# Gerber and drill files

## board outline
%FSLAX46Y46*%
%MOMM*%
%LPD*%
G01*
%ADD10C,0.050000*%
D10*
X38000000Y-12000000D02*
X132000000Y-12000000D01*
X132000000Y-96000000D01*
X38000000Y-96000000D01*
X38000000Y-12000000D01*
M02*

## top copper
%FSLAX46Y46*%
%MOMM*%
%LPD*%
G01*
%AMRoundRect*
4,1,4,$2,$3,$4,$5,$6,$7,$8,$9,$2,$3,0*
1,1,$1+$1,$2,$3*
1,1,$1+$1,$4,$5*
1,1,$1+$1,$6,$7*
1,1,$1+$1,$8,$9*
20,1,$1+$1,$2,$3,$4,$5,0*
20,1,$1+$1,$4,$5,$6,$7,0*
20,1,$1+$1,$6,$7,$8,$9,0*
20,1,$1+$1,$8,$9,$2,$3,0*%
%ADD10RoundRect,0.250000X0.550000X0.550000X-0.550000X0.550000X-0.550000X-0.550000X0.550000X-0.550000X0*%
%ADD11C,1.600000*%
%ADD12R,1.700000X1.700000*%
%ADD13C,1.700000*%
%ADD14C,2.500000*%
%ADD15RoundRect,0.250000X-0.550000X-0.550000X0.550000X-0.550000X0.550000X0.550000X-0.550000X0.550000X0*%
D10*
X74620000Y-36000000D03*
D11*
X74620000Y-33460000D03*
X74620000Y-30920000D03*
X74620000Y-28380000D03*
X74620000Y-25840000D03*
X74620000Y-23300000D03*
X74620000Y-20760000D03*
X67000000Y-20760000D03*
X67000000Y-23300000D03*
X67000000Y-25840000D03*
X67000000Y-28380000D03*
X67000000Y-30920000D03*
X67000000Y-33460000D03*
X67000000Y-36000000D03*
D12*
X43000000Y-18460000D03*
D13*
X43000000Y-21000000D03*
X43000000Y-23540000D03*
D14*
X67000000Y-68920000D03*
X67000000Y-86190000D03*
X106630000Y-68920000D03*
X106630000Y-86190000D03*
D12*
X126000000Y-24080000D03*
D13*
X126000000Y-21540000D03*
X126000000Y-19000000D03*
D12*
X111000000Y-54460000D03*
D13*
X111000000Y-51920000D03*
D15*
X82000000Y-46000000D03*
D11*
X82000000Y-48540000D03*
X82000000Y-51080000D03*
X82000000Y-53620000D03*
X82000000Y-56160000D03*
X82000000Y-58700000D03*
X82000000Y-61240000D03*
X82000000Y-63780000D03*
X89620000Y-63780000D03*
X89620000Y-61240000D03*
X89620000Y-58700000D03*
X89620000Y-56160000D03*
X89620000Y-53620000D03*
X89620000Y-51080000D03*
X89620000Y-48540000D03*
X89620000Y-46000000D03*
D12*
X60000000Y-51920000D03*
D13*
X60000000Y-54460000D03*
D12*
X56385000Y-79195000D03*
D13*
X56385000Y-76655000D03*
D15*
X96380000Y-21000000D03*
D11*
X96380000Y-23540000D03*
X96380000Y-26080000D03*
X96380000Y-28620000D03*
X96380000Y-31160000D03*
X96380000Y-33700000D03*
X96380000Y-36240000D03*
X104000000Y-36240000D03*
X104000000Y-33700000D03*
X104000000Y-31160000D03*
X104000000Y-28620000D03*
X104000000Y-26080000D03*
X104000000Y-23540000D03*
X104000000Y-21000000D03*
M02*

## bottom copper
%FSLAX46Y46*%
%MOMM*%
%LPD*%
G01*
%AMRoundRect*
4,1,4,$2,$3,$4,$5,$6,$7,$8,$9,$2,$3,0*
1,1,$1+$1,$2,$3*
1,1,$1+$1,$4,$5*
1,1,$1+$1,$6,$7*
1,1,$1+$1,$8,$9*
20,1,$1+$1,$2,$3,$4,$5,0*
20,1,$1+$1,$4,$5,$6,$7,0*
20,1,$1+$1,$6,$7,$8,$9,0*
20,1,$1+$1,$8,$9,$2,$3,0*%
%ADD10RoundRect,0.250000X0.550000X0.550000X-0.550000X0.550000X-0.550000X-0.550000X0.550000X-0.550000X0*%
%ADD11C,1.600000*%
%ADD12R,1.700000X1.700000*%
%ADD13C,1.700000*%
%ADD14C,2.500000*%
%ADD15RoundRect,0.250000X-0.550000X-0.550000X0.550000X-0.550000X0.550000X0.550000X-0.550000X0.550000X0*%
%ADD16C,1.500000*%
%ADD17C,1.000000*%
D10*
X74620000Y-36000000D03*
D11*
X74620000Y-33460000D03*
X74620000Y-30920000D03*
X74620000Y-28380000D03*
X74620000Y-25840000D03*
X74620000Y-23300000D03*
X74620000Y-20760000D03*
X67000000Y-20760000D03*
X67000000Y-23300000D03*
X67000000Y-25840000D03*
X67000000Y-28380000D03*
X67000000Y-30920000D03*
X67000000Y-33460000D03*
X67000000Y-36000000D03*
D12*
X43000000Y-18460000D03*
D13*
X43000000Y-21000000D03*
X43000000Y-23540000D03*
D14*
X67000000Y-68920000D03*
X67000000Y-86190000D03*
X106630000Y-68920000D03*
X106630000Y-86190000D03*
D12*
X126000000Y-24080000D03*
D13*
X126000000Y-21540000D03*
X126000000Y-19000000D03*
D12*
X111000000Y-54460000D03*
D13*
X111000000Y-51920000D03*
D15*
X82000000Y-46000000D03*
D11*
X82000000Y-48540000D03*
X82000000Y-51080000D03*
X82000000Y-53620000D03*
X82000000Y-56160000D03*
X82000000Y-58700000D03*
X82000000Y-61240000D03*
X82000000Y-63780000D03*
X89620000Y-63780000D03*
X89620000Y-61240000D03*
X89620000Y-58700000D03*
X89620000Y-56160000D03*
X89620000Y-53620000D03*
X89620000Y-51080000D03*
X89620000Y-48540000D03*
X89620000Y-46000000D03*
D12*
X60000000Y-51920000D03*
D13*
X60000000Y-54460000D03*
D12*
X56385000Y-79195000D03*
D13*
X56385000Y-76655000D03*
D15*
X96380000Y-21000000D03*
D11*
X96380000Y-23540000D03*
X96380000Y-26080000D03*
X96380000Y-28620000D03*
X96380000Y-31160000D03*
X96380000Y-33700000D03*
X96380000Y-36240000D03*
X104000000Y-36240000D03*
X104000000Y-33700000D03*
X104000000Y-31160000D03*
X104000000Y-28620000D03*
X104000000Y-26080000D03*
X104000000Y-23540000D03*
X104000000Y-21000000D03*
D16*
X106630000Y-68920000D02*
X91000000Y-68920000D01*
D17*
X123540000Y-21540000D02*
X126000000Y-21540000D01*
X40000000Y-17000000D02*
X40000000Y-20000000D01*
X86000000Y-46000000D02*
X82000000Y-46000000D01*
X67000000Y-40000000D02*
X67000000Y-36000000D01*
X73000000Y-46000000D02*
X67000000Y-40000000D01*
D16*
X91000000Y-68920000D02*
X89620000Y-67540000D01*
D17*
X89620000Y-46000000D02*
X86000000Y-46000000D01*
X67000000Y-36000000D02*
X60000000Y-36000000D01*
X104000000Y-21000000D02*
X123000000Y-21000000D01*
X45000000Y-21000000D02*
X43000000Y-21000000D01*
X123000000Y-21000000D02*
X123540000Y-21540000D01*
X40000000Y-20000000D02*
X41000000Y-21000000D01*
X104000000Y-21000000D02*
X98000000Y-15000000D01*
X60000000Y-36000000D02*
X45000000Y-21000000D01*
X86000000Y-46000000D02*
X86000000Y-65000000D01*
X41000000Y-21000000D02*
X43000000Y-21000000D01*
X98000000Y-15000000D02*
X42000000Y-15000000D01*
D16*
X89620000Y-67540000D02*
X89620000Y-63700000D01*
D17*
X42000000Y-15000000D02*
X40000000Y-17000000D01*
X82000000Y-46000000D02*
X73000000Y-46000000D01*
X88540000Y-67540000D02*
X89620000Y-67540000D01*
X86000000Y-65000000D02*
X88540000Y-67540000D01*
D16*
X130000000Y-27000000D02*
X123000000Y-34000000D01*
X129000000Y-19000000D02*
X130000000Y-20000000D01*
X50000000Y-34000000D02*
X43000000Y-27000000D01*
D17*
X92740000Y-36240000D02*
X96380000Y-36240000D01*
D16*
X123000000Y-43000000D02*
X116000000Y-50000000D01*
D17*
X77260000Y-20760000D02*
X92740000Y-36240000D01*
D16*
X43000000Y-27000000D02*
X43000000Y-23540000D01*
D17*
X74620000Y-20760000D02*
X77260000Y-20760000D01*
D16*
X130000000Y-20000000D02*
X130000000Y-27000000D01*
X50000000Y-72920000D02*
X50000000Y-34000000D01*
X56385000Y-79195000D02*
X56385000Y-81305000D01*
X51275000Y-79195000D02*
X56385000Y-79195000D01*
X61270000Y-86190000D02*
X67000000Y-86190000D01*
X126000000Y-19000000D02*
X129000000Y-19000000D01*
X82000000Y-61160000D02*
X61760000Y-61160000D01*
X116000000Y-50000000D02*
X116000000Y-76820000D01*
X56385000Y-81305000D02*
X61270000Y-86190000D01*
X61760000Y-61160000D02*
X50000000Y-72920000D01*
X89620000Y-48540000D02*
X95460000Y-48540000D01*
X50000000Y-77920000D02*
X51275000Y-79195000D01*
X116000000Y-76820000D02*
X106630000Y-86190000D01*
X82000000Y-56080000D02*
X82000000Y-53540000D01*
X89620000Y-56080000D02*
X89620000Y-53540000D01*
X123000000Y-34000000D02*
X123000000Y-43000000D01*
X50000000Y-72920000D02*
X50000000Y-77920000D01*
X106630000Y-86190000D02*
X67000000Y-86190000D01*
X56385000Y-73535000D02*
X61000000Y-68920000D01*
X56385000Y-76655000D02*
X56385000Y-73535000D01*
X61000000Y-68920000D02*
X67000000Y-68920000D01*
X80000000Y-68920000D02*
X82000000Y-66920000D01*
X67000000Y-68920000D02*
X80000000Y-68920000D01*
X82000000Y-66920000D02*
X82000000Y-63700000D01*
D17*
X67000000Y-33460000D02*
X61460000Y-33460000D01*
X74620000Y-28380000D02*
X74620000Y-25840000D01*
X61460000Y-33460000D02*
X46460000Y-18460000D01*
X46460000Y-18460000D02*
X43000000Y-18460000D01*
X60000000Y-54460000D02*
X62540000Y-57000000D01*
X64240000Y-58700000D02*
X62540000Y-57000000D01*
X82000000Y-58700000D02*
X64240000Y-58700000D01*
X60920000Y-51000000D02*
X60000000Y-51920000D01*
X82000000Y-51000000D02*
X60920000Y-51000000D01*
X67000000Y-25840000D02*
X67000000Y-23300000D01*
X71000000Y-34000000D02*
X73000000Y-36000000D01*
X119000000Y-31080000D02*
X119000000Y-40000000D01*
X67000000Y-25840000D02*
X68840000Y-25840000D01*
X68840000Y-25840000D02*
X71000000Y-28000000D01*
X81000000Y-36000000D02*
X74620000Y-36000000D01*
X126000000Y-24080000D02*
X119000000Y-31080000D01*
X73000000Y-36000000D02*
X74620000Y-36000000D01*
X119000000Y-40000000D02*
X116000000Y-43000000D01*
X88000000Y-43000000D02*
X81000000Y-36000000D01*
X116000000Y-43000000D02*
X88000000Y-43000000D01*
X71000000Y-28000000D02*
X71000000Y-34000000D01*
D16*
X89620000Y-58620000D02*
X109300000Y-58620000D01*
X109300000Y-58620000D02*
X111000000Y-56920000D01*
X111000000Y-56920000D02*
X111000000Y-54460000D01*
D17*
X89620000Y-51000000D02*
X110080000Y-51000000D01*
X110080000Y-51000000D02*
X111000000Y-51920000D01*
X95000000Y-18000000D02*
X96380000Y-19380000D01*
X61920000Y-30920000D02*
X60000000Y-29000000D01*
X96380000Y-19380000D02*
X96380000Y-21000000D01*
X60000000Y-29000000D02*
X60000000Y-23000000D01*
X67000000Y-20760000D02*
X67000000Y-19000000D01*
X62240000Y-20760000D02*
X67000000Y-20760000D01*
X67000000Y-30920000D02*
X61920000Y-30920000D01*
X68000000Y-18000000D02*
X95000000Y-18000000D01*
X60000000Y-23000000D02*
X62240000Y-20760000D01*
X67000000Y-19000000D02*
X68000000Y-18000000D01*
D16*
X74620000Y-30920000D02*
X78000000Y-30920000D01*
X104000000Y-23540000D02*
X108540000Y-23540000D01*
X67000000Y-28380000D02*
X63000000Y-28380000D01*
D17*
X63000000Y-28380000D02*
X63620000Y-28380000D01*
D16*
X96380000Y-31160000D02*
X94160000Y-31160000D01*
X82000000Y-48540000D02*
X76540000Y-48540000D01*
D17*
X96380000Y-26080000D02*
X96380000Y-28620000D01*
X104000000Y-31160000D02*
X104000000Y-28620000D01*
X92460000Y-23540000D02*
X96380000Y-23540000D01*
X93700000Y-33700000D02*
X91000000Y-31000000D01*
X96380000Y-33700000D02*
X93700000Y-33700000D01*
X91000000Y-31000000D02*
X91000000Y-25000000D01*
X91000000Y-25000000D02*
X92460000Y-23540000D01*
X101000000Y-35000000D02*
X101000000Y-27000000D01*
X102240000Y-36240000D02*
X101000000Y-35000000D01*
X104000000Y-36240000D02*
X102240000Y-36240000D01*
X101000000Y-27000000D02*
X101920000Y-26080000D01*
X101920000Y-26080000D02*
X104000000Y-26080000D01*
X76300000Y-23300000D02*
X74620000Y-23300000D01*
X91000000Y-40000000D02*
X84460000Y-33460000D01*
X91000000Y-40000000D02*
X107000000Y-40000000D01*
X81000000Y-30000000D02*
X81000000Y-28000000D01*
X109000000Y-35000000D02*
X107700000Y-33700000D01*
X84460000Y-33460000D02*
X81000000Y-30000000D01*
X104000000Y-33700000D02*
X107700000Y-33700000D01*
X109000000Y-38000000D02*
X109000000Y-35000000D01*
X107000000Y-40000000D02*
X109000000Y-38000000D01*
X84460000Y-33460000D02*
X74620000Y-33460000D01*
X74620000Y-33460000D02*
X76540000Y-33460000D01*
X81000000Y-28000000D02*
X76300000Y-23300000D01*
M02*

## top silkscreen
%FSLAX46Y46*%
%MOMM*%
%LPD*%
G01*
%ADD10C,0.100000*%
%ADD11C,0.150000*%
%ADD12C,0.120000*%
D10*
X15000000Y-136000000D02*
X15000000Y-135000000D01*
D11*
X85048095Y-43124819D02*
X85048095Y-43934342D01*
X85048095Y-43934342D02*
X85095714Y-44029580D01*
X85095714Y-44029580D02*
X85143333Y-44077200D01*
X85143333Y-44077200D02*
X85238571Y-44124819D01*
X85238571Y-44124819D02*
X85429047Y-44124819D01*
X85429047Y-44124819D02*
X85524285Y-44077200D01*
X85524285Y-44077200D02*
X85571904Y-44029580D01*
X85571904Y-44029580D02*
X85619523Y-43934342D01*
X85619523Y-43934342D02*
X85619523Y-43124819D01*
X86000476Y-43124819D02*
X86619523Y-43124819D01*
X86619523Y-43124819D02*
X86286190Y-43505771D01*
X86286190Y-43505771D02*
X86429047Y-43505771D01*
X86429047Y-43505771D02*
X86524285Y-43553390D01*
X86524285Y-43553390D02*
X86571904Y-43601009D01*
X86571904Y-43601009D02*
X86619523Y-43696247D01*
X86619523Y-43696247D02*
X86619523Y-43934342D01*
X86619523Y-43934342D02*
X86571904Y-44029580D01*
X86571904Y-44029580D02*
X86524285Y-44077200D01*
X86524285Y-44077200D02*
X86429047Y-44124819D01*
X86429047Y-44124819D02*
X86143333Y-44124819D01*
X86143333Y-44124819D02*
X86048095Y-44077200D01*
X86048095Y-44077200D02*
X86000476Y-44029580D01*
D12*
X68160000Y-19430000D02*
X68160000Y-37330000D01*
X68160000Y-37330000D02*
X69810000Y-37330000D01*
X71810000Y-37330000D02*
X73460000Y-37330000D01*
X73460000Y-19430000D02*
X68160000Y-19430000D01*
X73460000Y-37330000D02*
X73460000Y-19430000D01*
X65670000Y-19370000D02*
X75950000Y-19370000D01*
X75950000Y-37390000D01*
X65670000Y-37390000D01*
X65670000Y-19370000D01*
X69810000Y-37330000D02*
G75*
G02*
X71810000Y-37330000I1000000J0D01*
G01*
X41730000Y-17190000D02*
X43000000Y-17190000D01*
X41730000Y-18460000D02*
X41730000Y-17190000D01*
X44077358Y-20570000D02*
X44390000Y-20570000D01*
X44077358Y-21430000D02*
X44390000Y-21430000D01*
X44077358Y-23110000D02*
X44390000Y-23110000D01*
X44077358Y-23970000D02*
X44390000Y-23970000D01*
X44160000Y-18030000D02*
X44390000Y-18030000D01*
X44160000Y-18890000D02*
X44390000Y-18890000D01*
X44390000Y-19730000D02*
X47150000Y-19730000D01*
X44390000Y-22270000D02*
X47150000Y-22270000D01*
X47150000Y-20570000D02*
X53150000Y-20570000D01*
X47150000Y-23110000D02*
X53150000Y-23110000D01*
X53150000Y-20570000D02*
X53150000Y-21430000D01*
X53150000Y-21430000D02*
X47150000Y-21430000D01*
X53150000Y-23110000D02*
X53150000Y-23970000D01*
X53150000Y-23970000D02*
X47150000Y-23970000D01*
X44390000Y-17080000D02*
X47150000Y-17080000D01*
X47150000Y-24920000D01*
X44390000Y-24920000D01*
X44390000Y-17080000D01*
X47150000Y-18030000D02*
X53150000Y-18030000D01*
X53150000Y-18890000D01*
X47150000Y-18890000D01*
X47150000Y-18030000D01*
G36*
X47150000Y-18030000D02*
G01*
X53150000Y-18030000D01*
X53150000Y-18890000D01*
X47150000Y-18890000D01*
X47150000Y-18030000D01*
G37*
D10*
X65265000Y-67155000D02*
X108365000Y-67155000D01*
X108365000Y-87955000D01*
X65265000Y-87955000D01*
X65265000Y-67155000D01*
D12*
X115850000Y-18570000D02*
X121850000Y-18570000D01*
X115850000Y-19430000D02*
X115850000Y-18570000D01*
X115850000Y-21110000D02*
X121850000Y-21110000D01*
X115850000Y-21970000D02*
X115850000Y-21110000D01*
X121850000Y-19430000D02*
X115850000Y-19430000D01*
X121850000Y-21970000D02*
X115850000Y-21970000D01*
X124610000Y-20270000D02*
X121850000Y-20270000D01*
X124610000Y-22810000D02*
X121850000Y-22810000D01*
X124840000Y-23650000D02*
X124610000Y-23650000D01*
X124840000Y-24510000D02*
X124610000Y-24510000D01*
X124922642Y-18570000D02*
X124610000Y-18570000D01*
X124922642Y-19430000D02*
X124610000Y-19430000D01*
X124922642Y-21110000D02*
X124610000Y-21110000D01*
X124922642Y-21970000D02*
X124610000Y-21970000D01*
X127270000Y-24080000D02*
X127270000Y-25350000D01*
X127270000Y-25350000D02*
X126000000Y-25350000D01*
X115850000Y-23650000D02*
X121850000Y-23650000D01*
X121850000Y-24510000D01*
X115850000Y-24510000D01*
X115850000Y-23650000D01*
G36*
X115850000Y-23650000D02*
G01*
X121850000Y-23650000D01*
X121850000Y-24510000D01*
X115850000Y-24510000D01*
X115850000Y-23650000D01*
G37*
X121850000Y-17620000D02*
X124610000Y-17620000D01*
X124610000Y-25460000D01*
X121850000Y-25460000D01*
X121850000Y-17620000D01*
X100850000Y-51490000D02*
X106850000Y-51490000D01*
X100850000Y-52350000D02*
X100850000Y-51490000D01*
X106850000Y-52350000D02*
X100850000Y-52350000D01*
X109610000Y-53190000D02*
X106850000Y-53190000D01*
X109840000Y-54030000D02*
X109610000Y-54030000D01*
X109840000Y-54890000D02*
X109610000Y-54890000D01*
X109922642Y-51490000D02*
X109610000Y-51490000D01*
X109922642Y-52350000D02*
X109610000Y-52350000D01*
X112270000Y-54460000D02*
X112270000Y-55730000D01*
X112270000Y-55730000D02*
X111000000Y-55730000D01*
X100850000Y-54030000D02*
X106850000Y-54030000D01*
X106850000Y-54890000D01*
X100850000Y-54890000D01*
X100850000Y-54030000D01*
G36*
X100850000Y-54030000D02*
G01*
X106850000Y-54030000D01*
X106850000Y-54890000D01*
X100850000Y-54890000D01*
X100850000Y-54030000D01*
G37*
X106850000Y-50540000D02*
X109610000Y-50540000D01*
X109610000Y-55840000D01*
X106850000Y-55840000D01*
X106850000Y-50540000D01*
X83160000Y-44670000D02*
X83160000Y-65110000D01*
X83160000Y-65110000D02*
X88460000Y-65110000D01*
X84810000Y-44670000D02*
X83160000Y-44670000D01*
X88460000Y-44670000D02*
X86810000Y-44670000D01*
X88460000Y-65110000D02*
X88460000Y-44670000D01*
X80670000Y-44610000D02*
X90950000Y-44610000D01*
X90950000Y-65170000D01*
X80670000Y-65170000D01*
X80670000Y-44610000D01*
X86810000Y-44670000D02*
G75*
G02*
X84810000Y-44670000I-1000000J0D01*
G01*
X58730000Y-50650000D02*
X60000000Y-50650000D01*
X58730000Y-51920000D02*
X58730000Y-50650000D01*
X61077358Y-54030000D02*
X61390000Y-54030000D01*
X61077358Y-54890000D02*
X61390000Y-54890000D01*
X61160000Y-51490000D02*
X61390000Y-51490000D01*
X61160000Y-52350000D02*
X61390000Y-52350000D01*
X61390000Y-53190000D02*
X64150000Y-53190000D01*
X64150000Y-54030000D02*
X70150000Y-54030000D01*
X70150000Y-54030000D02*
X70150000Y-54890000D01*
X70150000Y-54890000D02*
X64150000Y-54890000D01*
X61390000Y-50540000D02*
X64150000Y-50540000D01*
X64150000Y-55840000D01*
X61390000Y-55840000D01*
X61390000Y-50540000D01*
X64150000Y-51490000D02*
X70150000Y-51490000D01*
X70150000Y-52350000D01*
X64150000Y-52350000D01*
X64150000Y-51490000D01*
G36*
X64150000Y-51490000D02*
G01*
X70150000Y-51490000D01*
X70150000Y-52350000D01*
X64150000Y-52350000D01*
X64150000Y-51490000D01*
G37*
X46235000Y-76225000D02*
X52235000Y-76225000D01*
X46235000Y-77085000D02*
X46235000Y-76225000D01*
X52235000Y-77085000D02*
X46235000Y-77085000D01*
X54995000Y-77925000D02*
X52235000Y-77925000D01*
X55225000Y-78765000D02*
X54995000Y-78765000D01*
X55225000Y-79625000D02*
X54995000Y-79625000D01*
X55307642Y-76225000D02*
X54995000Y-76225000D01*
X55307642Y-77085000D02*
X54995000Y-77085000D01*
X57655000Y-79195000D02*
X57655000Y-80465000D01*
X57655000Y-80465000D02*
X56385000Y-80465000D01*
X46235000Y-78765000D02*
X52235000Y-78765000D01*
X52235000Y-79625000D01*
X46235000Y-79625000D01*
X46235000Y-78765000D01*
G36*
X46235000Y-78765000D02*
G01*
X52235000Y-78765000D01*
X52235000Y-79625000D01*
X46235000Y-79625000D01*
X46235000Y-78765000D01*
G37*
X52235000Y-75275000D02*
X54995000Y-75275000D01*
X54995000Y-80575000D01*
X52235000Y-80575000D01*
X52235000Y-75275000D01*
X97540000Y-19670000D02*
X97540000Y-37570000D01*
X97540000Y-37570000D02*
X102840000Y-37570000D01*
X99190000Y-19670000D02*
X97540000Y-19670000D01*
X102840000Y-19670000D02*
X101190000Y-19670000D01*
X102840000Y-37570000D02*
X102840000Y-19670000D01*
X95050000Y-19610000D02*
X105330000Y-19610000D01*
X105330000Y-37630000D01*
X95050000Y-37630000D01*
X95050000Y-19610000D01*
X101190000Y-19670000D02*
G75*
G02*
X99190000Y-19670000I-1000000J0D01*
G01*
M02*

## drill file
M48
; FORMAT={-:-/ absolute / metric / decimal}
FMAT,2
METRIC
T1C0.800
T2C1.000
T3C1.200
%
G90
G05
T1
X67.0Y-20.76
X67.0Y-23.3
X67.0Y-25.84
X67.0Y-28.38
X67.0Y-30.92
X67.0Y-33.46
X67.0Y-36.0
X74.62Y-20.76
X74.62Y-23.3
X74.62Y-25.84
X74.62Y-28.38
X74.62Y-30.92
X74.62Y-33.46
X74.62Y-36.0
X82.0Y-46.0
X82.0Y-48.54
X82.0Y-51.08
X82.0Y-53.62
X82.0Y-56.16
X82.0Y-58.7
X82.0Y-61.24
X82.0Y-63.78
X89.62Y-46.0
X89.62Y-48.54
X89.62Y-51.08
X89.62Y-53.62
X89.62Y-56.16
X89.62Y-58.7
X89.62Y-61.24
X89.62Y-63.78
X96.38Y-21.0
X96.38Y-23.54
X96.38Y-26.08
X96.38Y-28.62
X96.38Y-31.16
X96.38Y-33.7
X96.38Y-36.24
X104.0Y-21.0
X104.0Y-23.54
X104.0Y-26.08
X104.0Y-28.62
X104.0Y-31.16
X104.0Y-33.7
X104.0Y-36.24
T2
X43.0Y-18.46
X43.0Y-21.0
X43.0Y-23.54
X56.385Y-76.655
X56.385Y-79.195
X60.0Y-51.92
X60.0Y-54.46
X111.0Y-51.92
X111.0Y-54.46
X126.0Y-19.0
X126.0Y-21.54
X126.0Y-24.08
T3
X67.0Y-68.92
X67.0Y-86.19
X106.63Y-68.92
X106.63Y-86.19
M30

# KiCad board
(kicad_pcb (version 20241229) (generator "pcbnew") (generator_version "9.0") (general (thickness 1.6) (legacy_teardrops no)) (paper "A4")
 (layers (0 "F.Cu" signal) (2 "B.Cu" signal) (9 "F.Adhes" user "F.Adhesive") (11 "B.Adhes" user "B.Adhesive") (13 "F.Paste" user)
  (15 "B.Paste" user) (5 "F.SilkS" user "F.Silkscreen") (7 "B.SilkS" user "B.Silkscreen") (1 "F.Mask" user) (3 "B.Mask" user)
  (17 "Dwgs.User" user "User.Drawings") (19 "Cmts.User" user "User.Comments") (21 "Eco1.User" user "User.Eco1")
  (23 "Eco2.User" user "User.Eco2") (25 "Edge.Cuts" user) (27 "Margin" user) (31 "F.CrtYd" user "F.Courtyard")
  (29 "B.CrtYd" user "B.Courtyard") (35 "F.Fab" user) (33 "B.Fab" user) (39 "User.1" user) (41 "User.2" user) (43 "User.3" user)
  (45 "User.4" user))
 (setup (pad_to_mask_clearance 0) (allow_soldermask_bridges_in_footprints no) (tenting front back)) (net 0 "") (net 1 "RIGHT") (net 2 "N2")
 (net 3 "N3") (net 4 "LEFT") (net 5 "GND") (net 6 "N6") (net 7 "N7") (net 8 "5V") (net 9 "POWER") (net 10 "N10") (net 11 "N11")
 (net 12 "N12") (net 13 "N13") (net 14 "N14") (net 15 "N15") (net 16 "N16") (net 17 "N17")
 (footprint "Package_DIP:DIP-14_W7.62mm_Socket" (layer "F.Cu") (at 74.62 36 180)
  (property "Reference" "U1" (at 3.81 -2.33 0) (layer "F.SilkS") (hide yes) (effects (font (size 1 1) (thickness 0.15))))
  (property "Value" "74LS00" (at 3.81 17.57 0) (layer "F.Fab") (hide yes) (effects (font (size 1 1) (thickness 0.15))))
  (fp_line (start 6.46 16.57) (end 6.46 -1.33) (stroke (width 0.12) (type solid)) (layer "F.SilkS"))
  (fp_line (start 6.46 -1.33) (end 4.81 -1.33) (stroke (width 0.12) (type solid)) (layer "F.SilkS"))
  (fp_line (start 2.81 -1.33) (end 1.16 -1.33) (stroke (width 0.12) (type solid)) (layer "F.SilkS"))
  (fp_line (start 1.16 16.57) (end 6.46 16.57) (stroke (width 0.12) (type solid)) (layer "F.SilkS"))
  (fp_line (start 1.16 -1.33) (end 1.16 16.57) (stroke (width 0.12) (type solid)) (layer "F.SilkS"))
  (fp_rect (start -1.33 -1.39) (end 8.95 16.63) (stroke (width 0.12) (type solid)) (fill no) (layer "F.SilkS"))
  (fp_arc (start 4.81 -1.33) (mid 3.81 -0.33) (end 2.81 -1.33) (stroke (width 0.12) (type solid)) (layer "F.SilkS"))
  (pad "1" thru_hole roundrect (at 0 0 180) (size 1.6 1.6) (drill 0.8) (layers "*.Cu" "*.Mask") (remove_unused_layers no)
   (roundrect_rratio 0.15625) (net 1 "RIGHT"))
  (pad "2" thru_hole circle (at 0 2.54 180) (size 1.6 1.6) (drill 0.8) (layers "*.Cu" "*.Mask") (remove_unused_layers no) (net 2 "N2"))
  (pad "3" thru_hole circle (at 0 5.08 180) (size 1.6 1.6) (drill 0.8) (layers "*.Cu" "*.Mask") (remove_unused_layers no) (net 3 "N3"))
  (pad "4" thru_hole circle (at 0 7.62 180) (size 1.6 1.6) (drill 0.8) (layers "*.Cu" "*.Mask") (remove_unused_layers no) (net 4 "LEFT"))
  (pad "5" thru_hole circle (at 0 10.16 180) (size 1.6 1.6) (drill 0.8) (layers "*.Cu" "*.Mask") (remove_unused_layers no) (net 4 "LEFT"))
  (pad "6" thru_hole circle (at 0 12.7 180) (size 1.6 1.6) (drill 0.8) (layers "*.Cu" "*.Mask") (remove_unused_layers no) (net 2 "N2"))
  (pad "7" thru_hole circle (at 0 15.24 180) (size 1.6 1.6) (drill 0.8) (layers "*.Cu" "*.Mask") (remove_unused_layers no) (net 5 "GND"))
  (pad "8" thru_hole circle (at 7.62 15.24 180) (size 1.6 1.6) (drill 0.8) (layers "*.Cu" "*.Mask") (remove_unused_layers no) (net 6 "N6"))
  (pad "9" thru_hole circle (at 7.62 12.7 180) (size 1.6 1.6) (drill 0.8) (layers "*.Cu" "*.Mask") (remove_unused_layers no) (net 1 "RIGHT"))
  (pad "10" thru_hole circle (at 7.62 10.16 180) (size 1.6 1.6) (drill 0.8) (layers "*.Cu" "*.Mask") (remove_unused_layers no)
   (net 1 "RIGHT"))
  (pad "11" thru_hole circle (at 7.62 7.62 180) (size 1.6 1.6) (drill 0.8) (layers "*.Cu" "*.Mask") (remove_unused_layers no) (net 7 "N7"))
  (pad "12" thru_hole circle (at 7.62 5.08 180) (size 1.6 1.6) (drill 0.8) (layers "*.Cu" "*.Mask") (remove_unused_layers no) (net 6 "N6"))
  (pad "13" thru_hole circle (at 7.62 2.54 180) (size 1.6 1.6) (drill 0.8) (layers "*.Cu" "*.Mask") (remove_unused_layers no) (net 4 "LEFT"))
  (pad "14" thru_hole circle (at 7.62 0 180) (size 1.6 1.6) (drill 0.8) (layers "*.Cu" "*.Mask") (remove_unused_layers no) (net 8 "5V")))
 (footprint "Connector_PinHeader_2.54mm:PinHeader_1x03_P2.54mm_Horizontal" (layer "F.Cu") (at 43 18.46)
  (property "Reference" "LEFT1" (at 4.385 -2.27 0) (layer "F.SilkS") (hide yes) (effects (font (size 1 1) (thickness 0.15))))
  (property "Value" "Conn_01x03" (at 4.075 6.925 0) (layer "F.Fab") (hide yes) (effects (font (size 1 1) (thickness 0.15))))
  (fp_line (start -1.27 -1.27) (end 0 -1.27) (stroke (width 0.12) (type solid)) (layer "F.SilkS"))
  (fp_line (start -1.27 0) (end -1.27 -1.27) (stroke (width 0.12) (type solid)) (layer "F.SilkS"))
  (fp_line (start 1.077358 2.11) (end 1.39 2.11) (stroke (width 0.12) (type solid)) (layer "F.SilkS"))
  (fp_line (start 1.077358 2.97) (end 1.39 2.97) (stroke (width 0.12) (type solid)) (layer "F.SilkS"))
  (fp_line (start 1.077358 4.65) (end 1.39 4.65) (stroke (width 0.12) (type solid)) (layer "F.SilkS"))
  (fp_line (start 1.077358 5.51) (end 1.39 5.51) (stroke (width 0.12) (type solid)) (layer "F.SilkS"))
  (fp_line (start 1.16 -0.43) (end 1.39 -0.43) (stroke (width 0.12) (type solid)) (layer "F.SilkS"))
  (fp_line (start 1.16 0.43) (end 1.39 0.43) (stroke (width 0.12) (type solid)) (layer "F.SilkS"))
  (fp_line (start 1.39 1.27) (end 4.15 1.27) (stroke (width 0.12) (type solid)) (layer "F.SilkS"))
  (fp_line (start 1.39 3.81) (end 4.15 3.81) (stroke (width 0.12) (type solid)) (layer "F.SilkS"))
  (fp_line (start 4.15 2.11) (end 10.15 2.11) (stroke (width 0.12) (type solid)) (layer "F.SilkS"))
  (fp_line (start 4.15 4.65) (end 10.15 4.65) (stroke (width 0.12) (type solid)) (layer "F.SilkS"))
  (fp_line (start 10.15 2.11) (end 10.15 2.97) (stroke (width 0.12) (type solid)) (layer "F.SilkS"))
  (fp_line (start 10.15 2.97) (end 4.15 2.97) (stroke (width 0.12) (type solid)) (layer "F.SilkS"))
  (fp_line (start 10.15 4.65) (end 10.15 5.51) (stroke (width 0.12) (type solid)) (layer "F.SilkS"))
  (fp_line (start 10.15 5.51) (end 4.15 5.51) (stroke (width 0.12) (type solid)) (layer "F.SilkS"))
  (fp_rect (start 1.39 -1.38) (end 4.15 6.46) (stroke (width 0.12) (type solid)) (fill no) (layer "F.SilkS"))
  (fp_rect (start 4.15 -0.43) (end 10.15 0.43) (stroke (width 0.12) (type solid)) (fill yes) (layer "F.SilkS"))
  (pad "1" thru_hole rect (at 0 0) (size 1.7 1.7) (drill 1) (layers "*.Cu" "*.Mask") (remove_unused_layers no) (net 4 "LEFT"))
  (pad "2" thru_hole circle (at 0 2.54) (size 1.7 1.7) (drill 1) (layers "*.Cu" "*.Mask") (remove_unused_layers no) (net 8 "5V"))
  (pad "3" thru_hole circle (at 0 5.08) (size 1.7 1.7) (drill 1) (layers "*.Cu" "*.Mask") (remove_unused_layers no) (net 5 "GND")))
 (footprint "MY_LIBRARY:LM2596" (layer "F.Cu") (at 67 86.19)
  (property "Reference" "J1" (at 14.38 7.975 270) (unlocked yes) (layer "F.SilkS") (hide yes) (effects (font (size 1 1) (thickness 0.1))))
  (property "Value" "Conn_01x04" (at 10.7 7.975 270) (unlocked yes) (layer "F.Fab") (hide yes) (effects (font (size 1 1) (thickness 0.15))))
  (fp_rect (start -1.735 1.765) (end 41.365 -19.035) (stroke (width 0.1) (type solid)) (fill no) (layer "F.SilkS"))
  (pad "IN+" thru_hole circle (at 0 -17.27) (size 2.5 2.5) (drill 1.2) (layers "*.Cu" "*.Mask") (remove_unused_layers no) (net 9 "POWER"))
  (pad "IN-" thru_hole circle (at 0 0) (size 2.5 2.5) (drill 1.2) (layers "*.Cu" "*.Mask") (remove_unused_layers no) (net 5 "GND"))
  (pad "OUT+" thru_hole circle (at 39.63 -17.27) (size 2.5 2.5) (drill 1.2) (layers "*.Cu" "*.Mask") (remove_unused_layers no) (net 8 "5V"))
  (pad "OUT-" thru_hole circle (at 39.63 0) (size 2.5 2.5) (drill 1.2) (layers "*.Cu" "*.Mask") (remove_unused_layers no) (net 5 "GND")))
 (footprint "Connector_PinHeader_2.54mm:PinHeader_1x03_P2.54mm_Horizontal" (layer "F.Cu") (at 126 24.08 180)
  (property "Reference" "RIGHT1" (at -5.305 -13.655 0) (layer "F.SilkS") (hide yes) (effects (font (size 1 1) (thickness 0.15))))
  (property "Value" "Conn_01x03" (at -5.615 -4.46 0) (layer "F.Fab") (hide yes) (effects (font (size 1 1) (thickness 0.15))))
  (fp_line (start 10.15 5.51) (end 4.15 5.51) (stroke (width 0.12) (type solid)) (layer "F.SilkS"))
  (fp_line (start 10.15 4.65) (end 10.15 5.51) (stroke (width 0.12) (type solid)) (layer "F.SilkS"))
  (fp_line (start 10.15 2.97) (end 4.15 2.97) (stroke (width 0.12) (type solid)) (layer "F.SilkS"))
  (fp_line (start 10.15 2.11) (end 10.15 2.97) (stroke (width 0.12) (type solid)) (layer "F.SilkS"))
  (fp_line (start 4.15 4.65) (end 10.15 4.65) (stroke (width 0.12) (type solid)) (layer "F.SilkS"))
  (fp_line (start 4.15 2.11) (end 10.15 2.11) (stroke (width 0.12) (type solid)) (layer "F.SilkS"))
  (fp_line (start 1.39 3.81) (end 4.15 3.81) (stroke (width 0.12) (type solid)) (layer "F.SilkS"))
  (fp_line (start 1.39 1.27) (end 4.15 1.27) (stroke (width 0.12) (type solid)) (layer "F.SilkS"))
  (fp_line (start 1.16 0.43) (end 1.39 0.43) (stroke (width 0.12) (type solid)) (layer "F.SilkS"))
  (fp_line (start 1.16 -0.43) (end 1.39 -0.43) (stroke (width 0.12) (type solid)) (layer "F.SilkS"))
  (fp_line (start 1.077358 5.51) (end 1.39 5.51) (stroke (width 0.12) (type solid)) (layer "F.SilkS"))
  (fp_line (start 1.077358 4.65) (end 1.39 4.65) (stroke (width 0.12) (type solid)) (layer "F.SilkS"))
  (fp_line (start 1.077358 2.97) (end 1.39 2.97) (stroke (width 0.12) (type solid)) (layer "F.SilkS"))
  (fp_line (start 1.077358 2.11) (end 1.39 2.11) (stroke (width 0.12) (type solid)) (layer "F.SilkS"))
  (fp_line (start -1.27 0) (end -1.27 -1.27) (stroke (width 0.12) (type solid)) (layer "F.SilkS"))
  (fp_line (start -1.27 -1.27) (end 0 -1.27) (stroke (width 0.12) (type solid)) (layer "F.SilkS"))
  (fp_rect (start 4.15 -0.43) (end 10.15 0.43) (stroke (width 0.12) (type solid)) (fill yes) (layer "F.SilkS"))
  (fp_rect (start 1.39 -1.38) (end 4.15 6.46) (stroke (width 0.12) (type solid)) (fill no) (layer "F.SilkS"))
  (pad "1" thru_hole rect (at 0 0 180) (size 1.7 1.7) (drill 1) (layers "*.Cu" "*.Mask") (remove_unused_layers no) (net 1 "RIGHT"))
  (pad "2" thru_hole circle (at 0 2.54 180) (size 1.7 1.7) (drill 1) (layers "*.Cu" "*.Mask") (remove_unused_layers no) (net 8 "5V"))
  (pad "3" thru_hole circle (at 0 5.08 180) (size 1.7 1.7) (drill 1) (layers "*.Cu" "*.Mask") (remove_unused_layers no) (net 5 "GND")))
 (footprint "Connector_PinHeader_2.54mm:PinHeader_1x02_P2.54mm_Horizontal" (layer "F.Cu") (at 111 54.46 180)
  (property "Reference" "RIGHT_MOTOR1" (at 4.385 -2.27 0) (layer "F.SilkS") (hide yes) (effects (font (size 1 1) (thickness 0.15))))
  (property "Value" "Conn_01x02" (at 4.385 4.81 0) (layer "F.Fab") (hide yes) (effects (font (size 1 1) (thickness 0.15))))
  (fp_line (start 10.15 2.97) (end 4.15 2.97) (stroke (width 0.12) (type solid)) (layer "F.SilkS"))
  (fp_line (start 10.15 2.11) (end 10.15 2.97) (stroke (width 0.12) (type solid)) (layer "F.SilkS"))
  (fp_line (start 4.15 2.11) (end 10.15 2.11) (stroke (width 0.12) (type solid)) (layer "F.SilkS"))
  (fp_line (start 1.39 1.27) (end 4.15 1.27) (stroke (width 0.12) (type solid)) (layer "F.SilkS"))
  (fp_line (start 1.16 0.43) (end 1.39 0.43) (stroke (width 0.12) (type solid)) (layer "F.SilkS"))
  (fp_line (start 1.16 -0.43) (end 1.39 -0.43) (stroke (width 0.12) (type solid)) (layer "F.SilkS"))
  (fp_line (start 1.077358 2.97) (end 1.39 2.97) (stroke (width 0.12) (type solid)) (layer "F.SilkS"))
  (fp_line (start 1.077358 2.11) (end 1.39 2.11) (stroke (width 0.12) (type solid)) (layer "F.SilkS"))
  (fp_line (start -1.27 0) (end -1.27 -1.27) (stroke (width 0.12) (type solid)) (layer "F.SilkS"))
  (fp_line (start -1.27 -1.27) (end 0 -1.27) (stroke (width 0.12) (type solid)) (layer "F.SilkS"))
  (fp_rect (start 4.15 -0.43) (end 10.15 0.43) (stroke (width 0.12) (type solid)) (fill yes) (layer "F.SilkS"))
  (fp_rect (start 1.39 -1.38) (end 4.15 3.92) (stroke (width 0.12) (type solid)) (fill no) (layer "F.SilkS"))
  (pad "1" thru_hole rect (at 0 0 180) (size 1.7 1.7) (drill 1) (layers "*.Cu" "*.Mask") (remove_unused_layers no) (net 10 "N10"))
  (pad "2" thru_hole circle (at 0 2.54 180) (size 1.7 1.7) (drill 1) (layers "*.Cu" "*.Mask") (remove_unused_layers no) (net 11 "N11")))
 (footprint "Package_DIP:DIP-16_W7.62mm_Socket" (layer "F.Cu") (at 82 46)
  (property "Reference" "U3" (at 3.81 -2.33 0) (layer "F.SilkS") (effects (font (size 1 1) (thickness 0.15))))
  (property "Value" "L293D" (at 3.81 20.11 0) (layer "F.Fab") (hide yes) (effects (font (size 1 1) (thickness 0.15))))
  (fp_line (start 1.16 -1.33) (end 1.16 19.11) (stroke (width 0.12) (type solid)) (layer "F.SilkS"))
  (fp_line (start 1.16 19.11) (end 6.46 19.11) (stroke (width 0.12) (type solid)) (layer "F.SilkS"))
  (fp_line (start 2.81 -1.33) (end 1.16 -1.33) (stroke (width 0.12) (type solid)) (layer "F.SilkS"))
  (fp_line (start 6.46 -1.33) (end 4.81 -1.33) (stroke (width 0.12) (type solid)) (layer "F.SilkS"))
  (fp_line (start 6.46 19.11) (end 6.46 -1.33) (stroke (width 0.12) (type solid)) (layer "F.SilkS"))
  (fp_rect (start -1.33 -1.39) (end 8.95 19.17) (stroke (width 0.12) (type solid)) (fill no) (layer "F.SilkS"))
  (fp_arc (start 4.81 -1.33) (mid 3.81 -0.33) (end 2.81 -1.33) (stroke (width 0.12) (type solid)) (layer "F.SilkS"))
  (pad "1" thru_hole roundrect (at 0 0) (size 1.6 1.6) (drill 0.8) (layers "*.Cu" "*.Mask") (remove_unused_layers no)
   (roundrect_rratio 0.15625) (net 8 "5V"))
  (pad "2" thru_hole circle (at 0 2.54) (size 1.6 1.6) (drill 0.8) (layers "*.Cu" "*.Mask") (remove_unused_layers no) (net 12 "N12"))
  (pad "3" thru_hole circle (at 0 5.08) (size 1.6 1.6) (drill 0.8) (layers "*.Cu" "*.Mask") (remove_unused_layers no) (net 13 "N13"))
  (pad "4" thru_hole circle (at 0 7.62) (size 1.6 1.6) (drill 0.8) (layers "*.Cu" "*.Mask") (remove_unused_layers no) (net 5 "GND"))
  (pad "5" thru_hole circle (at 0 10.16) (size 1.6 1.6) (drill 0.8) (layers "*.Cu" "*.Mask") (remove_unused_layers no) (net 5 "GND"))
  (pad "6" thru_hole circle (at 0 12.7) (size 1.6 1.6) (drill 0.8) (layers "*.Cu" "*.Mask") (remove_unused_layers no) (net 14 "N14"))
  (pad "7" thru_hole circle (at 0 15.24) (size 1.6 1.6) (drill 0.8) (layers "*.Cu" "*.Mask") (remove_unused_layers no) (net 5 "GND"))
  (pad "8" thru_hole circle (at 0 17.78) (size 1.6 1.6) (drill 0.8) (layers "*.Cu" "*.Mask") (remove_unused_layers no) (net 9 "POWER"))
  (pad "9" thru_hole circle (at 7.62 17.78) (size 1.6 1.6) (drill 0.8) (layers "*.Cu" "*.Mask") (remove_unused_layers no) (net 8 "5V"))
  (pad "10" thru_hole circle (at 7.62 15.24) (size 1.6 1.6) (drill 0.8) (layers "*.Cu" "*.Mask") (remove_unused_layers no) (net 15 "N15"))
  (pad "11" thru_hole circle (at 7.62 12.7) (size 1.6 1.6) (drill 0.8) (layers "*.Cu" "*.Mask") (remove_unused_layers no) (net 10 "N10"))
  (pad "12" thru_hole circle (at 7.62 10.16) (size 1.6 1.6) (drill 0.8) (layers "*.Cu" "*.Mask") (remove_unused_layers no) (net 5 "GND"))
  (pad "13" thru_hole circle (at 7.62 7.62) (size 1.6 1.6) (drill 0.8) (layers "*.Cu" "*.Mask") (remove_unused_layers no) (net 5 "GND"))
  (pad "14" thru_hole circle (at 7.62 5.08) (size 1.6 1.6) (drill 0.8) (layers "*.Cu" "*.Mask") (remove_unused_layers no) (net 11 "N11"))
  (pad "15" thru_hole circle (at 7.62 2.54) (size 1.6 1.6) (drill 0.8) (layers "*.Cu" "*.Mask") (remove_unused_layers no) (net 5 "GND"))
  (pad "16" thru_hole circle (at 7.62 0) (size 1.6 1.6) (drill 0.8) (layers "*.Cu" "*.Mask") (remove_unused_layers no) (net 8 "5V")))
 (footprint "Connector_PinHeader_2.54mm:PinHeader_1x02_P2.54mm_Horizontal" (layer "F.Cu") (at 60 51.92)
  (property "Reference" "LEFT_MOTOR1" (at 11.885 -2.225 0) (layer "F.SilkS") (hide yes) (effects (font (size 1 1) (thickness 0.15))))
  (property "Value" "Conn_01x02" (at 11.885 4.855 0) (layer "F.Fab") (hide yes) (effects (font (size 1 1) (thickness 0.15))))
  (fp_line (start -1.27 -1.27) (end 0 -1.27) (stroke (width 0.12) (type solid)) (layer "F.SilkS"))
  (fp_line (start -1.27 0) (end -1.27 -1.27) (stroke (width 0.12) (type solid)) (layer "F.SilkS"))
  (fp_line (start 1.077358 2.11) (end 1.39 2.11) (stroke (width 0.12) (type solid)) (layer "F.SilkS"))
  (fp_line (start 1.077358 2.97) (end 1.39 2.97) (stroke (width 0.12) (type solid)) (layer "F.SilkS"))
  (fp_line (start 1.16 -0.43) (end 1.39 -0.43) (stroke (width 0.12) (type solid)) (layer "F.SilkS"))
  (fp_line (start 1.16 0.43) (end 1.39 0.43) (stroke (width 0.12) (type solid)) (layer "F.SilkS"))
  (fp_line (start 1.39 1.27) (end 4.15 1.27) (stroke (width 0.12) (type solid)) (layer "F.SilkS"))
  (fp_line (start 4.15 2.11) (end 10.15 2.11) (stroke (width 0.12) (type solid)) (layer "F.SilkS"))
  (fp_line (start 10.15 2.11) (end 10.15 2.97) (stroke (width 0.12) (type solid)) (layer "F.SilkS"))
  (fp_line (start 10.15 2.97) (end 4.15 2.97) (stroke (width 0.12) (type solid)) (layer "F.SilkS"))
  (fp_rect (start 1.39 -1.38) (end 4.15 3.92) (stroke (width 0.12) (type solid)) (fill no) (layer "F.SilkS"))
  (fp_rect (start 4.15 -0.43) (end 10.15 0.43) (stroke (width 0.12) (type solid)) (fill yes) (layer "F.SilkS"))
  (pad "1" thru_hole rect (at 0 0) (size 1.7 1.7) (drill 1) (layers "*.Cu" "*.Mask") (remove_unused_layers no) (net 13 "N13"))
  (pad "2" thru_hole circle (at 0 2.54) (size 1.7 1.7) (drill 1) (layers "*.Cu" "*.Mask") (remove_unused_layers no) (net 14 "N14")))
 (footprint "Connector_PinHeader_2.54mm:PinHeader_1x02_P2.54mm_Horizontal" (layer "F.Cu") (at 56.385 79.195 180)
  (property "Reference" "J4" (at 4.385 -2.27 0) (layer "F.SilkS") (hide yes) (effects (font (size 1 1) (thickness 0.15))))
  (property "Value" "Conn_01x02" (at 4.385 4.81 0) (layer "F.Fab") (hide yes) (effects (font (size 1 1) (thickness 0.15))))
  (fp_line (start 10.15 2.97) (end 4.15 2.97) (stroke (width 0.12) (type solid)) (layer "F.SilkS"))
  (fp_line (start 10.15 2.11) (end 10.15 2.97) (stroke (width 0.12) (type solid)) (layer "F.SilkS"))
  (fp_line (start 4.15 2.11) (end 10.15 2.11) (stroke (width 0.12) (type solid)) (layer "F.SilkS"))
  (fp_line (start 1.39 1.27) (end 4.15 1.27) (stroke (width 0.12) (type solid)) (layer "F.SilkS"))
  (fp_line (start 1.16 0.43) (end 1.39 0.43) (stroke (width 0.12) (type solid)) (layer "F.SilkS"))
  (fp_line (start 1.16 -0.43) (end 1.39 -0.43) (stroke (width 0.12) (type solid)) (layer "F.SilkS"))
  (fp_line (start 1.077358 2.97) (end 1.39 2.97) (stroke (width 0.12) (type solid)) (layer "F.SilkS"))
  (fp_line (start 1.077358 2.11) (end 1.39 2.11) (stroke (width 0.12) (type solid)) (layer "F.SilkS"))
  (fp_line (start -1.27 0) (end -1.27 -1.27) (stroke (width 0.12) (type solid)) (layer "F.SilkS"))
  (fp_line (start -1.27 -1.27) (end 0 -1.27) (stroke (width 0.12) (type solid)) (layer "F.SilkS"))
  (fp_rect (start 4.15 -0.43) (end 10.15 0.43) (stroke (width 0.12) (type solid)) (fill yes) (layer "F.SilkS"))
  (fp_rect (start 1.39 -1.38) (end 4.15 3.92) (stroke (width 0.12) (type solid)) (fill no) (layer "F.SilkS"))
  (pad "1" thru_hole rect (at 0 0 180) (size 1.7 1.7) (drill 1) (layers "*.Cu" "*.Mask") (remove_unused_layers no) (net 5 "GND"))
  (pad "2" thru_hole circle (at 0 2.54 180) (size 1.7 1.7) (drill 1) (layers "*.Cu" "*.Mask") (remove_unused_layers no) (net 9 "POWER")))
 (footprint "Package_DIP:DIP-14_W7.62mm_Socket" (layer "F.Cu") (at 96.38 21)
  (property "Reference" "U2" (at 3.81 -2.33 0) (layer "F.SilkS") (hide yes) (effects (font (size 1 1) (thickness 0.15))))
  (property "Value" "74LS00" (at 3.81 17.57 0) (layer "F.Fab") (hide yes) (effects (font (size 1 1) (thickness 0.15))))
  (fp_line (start 1.16 -1.33) (end 1.16 16.57) (stroke (width 0.12) (type solid)) (layer "F.SilkS"))
  (fp_line (start 1.16 16.57) (end 6.46 16.57) (stroke (width 0.12) (type solid)) (layer "F.SilkS"))
  (fp_line (start 2.81 -1.33) (end 1.16 -1.33) (stroke (width 0.12) (type solid)) (layer "F.SilkS"))
  (fp_line (start 6.46 -1.33) (end 4.81 -1.33) (stroke (width 0.12) (type solid)) (layer "F.SilkS"))
  (fp_line (start 6.46 16.57) (end 6.46 -1.33) (stroke (width 0.12) (type solid)) (layer "F.SilkS"))
  (fp_rect (start -1.33 -1.39) (end 8.95 16.63) (stroke (width 0.12) (type solid)) (fill no) (layer "F.SilkS"))
  (fp_arc (start 4.81 -1.33) (mid 3.81 -0.33) (end 2.81 -1.33) (stroke (width 0.12) (type solid)) (layer "F.SilkS"))
  (pad "1" thru_hole roundrect (at 0 0) (size 1.6 1.6) (drill 0.8) (layers "*.Cu" "*.Mask") (remove_unused_layers no)
   (roundrect_rratio 0.15625) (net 6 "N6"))
  (pad "2" thru_hole circle (at 0 2.54) (size 1.6 1.6) (drill 0.8) (layers "*.Cu" "*.Mask") (remove_unused_layers no) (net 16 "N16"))
  (pad "3" thru_hole circle (at 0 5.08) (size 1.6 1.6) (drill 0.8) (layers "*.Cu" "*.Mask") (remove_unused_layers no) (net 12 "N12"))
  (pad "4" thru_hole circle (at 0 7.62) (size 1.6 1.6) (drill 0.8) (layers "*.Cu" "*.Mask") (remove_unused_layers no) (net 12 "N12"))
  (pad "5" thru_hole circle (at 0 10.16) (size 1.6 1.6) (drill 0.8) (layers "*.Cu" "*.Mask") (remove_unused_layers no) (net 7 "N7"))
  (pad "6" thru_hole circle (at 0 12.7) (size 1.6 1.6) (drill 0.8) (layers "*.Cu" "*.Mask") (remove_unused_layers no) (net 16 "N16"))
  (pad "7" thru_hole circle (at 0 15.24) (size 1.6 1.6) (drill 0.8) (layers "*.Cu" "*.Mask") (remove_unused_layers no) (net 5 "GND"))
  (pad "8" thru_hole circle (at 7.62 15.24) (size 1.6 1.6) (drill 0.8) (layers "*.Cu" "*.Mask") (remove_unused_layers no) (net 15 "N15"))
  (pad "9" thru_hole circle (at 7.62 12.7) (size 1.6 1.6) (drill 0.8) (layers "*.Cu" "*.Mask") (remove_unused_layers no) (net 2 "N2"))
  (pad "10" thru_hole circle (at 7.62 10.16) (size 1.6 1.6) (drill 0.8) (layers "*.Cu" "*.Mask") (remove_unused_layers no) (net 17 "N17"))
  (pad "11" thru_hole circle (at 7.62 7.62) (size 1.6 1.6) (drill 0.8) (layers "*.Cu" "*.Mask") (remove_unused_layers no) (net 17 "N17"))
  (pad "12" thru_hole circle (at 7.62 5.08) (size 1.6 1.6) (drill 0.8) (layers "*.Cu" "*.Mask") (remove_unused_layers no) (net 15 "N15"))
  (pad "13" thru_hole circle (at 7.62 2.54) (size 1.6 1.6) (drill 0.8) (layers "*.Cu" "*.Mask") (remove_unused_layers no) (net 3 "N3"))
  (pad "14" thru_hole circle (at 7.62 0) (size 1.6 1.6) (drill 0.8) (layers "*.Cu" "*.Mask") (remove_unused_layers no) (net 8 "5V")))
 (gr_line (start 15 136) (end 15 135) (stroke (width 0.1) (type default)) (layer "F.SilkS"))
 (gr_rect (start 38 12) (end 132 96) (stroke (width 0.05) (type default)) (fill no) (layer "Edge.Cuts"))
 (segment (start 106.63 68.92) (end 91 68.92) (width 1.5) (layer "B.Cu") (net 8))
 (segment (start 123.54 21.54) (end 126 21.54) (width 1) (layer "B.Cu") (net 8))
 (segment (start 40 17) (end 40 20) (width 1) (layer "B.Cu") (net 8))
 (segment (start 86 46) (end 82 46) (width 1) (layer "B.Cu") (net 8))
 (segment (start 67 40) (end 67 36) (width 1) (layer "B.Cu") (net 8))
 (segment (start 73 46) (end 67 40) (width 1) (layer "B.Cu") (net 8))
 (segment (start 91 68.92) (end 89.62 67.54) (width 1.5) (layer "B.Cu") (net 8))
 (segment (start 89.62 46) (end 86 46) (width 1) (layer "B.Cu") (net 8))
 (segment (start 67 36) (end 60 36) (width 1) (layer "B.Cu") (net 8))
 (segment (start 104 21) (end 123 21) (width 1) (layer "B.Cu") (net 8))
 (segment (start 45 21) (end 43 21) (width 1) (layer "B.Cu") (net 8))
 (segment (start 123 21) (end 123.54 21.54) (width 1) (layer "B.Cu") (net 8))
 (segment (start 40 20) (end 41 21) (width 1) (layer "B.Cu") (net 8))
 (segment (start 104 21) (end 98 15) (width 1) (layer "B.Cu") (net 8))
 (segment (start 60 36) (end 45 21) (width 1) (layer "B.Cu") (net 8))
 (segment (start 86 46) (end 86 65) (width 1) (layer "B.Cu") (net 8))
 (segment (start 41 21) (end 43 21) (width 1) (layer "B.Cu") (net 8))
 (segment (start 98 15) (end 42 15) (width 1) (layer "B.Cu") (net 8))
 (segment (start 89.62 67.54) (end 89.62 63.7) (width 1.5) (layer "B.Cu") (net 8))
 (segment (start 42 15) (end 40 17) (width 1) (layer "B.Cu") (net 8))
 (segment (start 82 46) (end 73 46) (width 1) (layer "B.Cu") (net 8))
 (segment (start 88.54 67.54) (end 89.62 67.54) (width 1) (layer "B.Cu") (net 8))
 (segment (start 86 65) (end 88.54 67.54) (width 1) (layer "B.Cu") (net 8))
 (segment (start 130 27) (end 123 34) (width 1.5) (layer "B.Cu") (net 5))
 (segment (start 129 19) (end 130 20) (width 1.5) (layer "B.Cu") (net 5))
 (segment (start 50 34) (end 43 27) (width 1.5) (layer "B.Cu") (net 5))
 (segment (start 92.74 36.24) (end 96.38 36.24) (width 1) (layer "B.Cu") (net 5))
 (segment (start 123 43) (end 116 50) (width 1.5) (layer "B.Cu") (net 5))
 (segment (start 77.26 20.76) (end 92.74 36.24) (width 1) (layer "B.Cu") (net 5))
 (segment (start 43 27) (end 43 23.54) (width 1.5) (layer "B.Cu") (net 5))
 (segment (start 74.62 20.76) (end 77.26 20.76) (width 1) (layer "B.Cu") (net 5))
 (segment (start 130 20) (end 130 27) (width 1.5) (layer "B.Cu") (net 5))
 (segment (start 50 72.92) (end 50 34) (width 1.5) (layer "B.Cu") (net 5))
 (segment (start 56.385 79.195) (end 56.385 81.305) (width 1.5) (layer "B.Cu") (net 5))
 (segment (start 51.275 79.195) (end 56.385 79.195) (width 1.5) (layer "B.Cu") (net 5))
 (segment (start 61.27 86.19) (end 67 86.19) (width 1.5) (layer "B.Cu") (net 5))
 (segment (start 126 19) (end 129 19) (width 1.5) (layer "B.Cu") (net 5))
 (segment (start 82 61.16) (end 61.76 61.16) (width 1.5) (layer "B.Cu") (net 5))
 (segment (start 116 50) (end 116 76.82) (width 1.5) (layer "B.Cu") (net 5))
 (segment (start 56.385 81.305) (end 61.27 86.19) (width 1.5) (layer "B.Cu") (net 5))
 (segment (start 61.76 61.16) (end 50 72.92) (width 1.5) (layer "B.Cu") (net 5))
 (segment (start 89.62 48.54) (end 95.46 48.54) (width 1.5) (layer "B.Cu") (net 5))
 (segment (start 50 77.92) (end 51.275 79.195) (width 1.5) (layer "B.Cu") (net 5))
 (segment (start 116 76.82) (end 106.63 86.19) (width 1.5) (layer "B.Cu") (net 5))
 (segment (start 82 56.08) (end 82 53.54) (width 1.5) (layer "B.Cu") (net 5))
 (segment (start 89.62 56.08) (end 89.62 53.54) (width 1.5) (layer "B.Cu") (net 5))
 (segment (start 123 34) (end 123 43) (width 1.5) (layer "B.Cu") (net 5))
 (segment (start 50 72.92) (end 50 77.92) (width 1.5) (layer "B.Cu") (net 5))
 (segment (start 106.63 86.19) (end 67 86.19) (width 1.5) (layer "B.Cu") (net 5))
 (segment (start 56.385 73.535) (end 61 68.92) (width 1.5) (layer "B.Cu") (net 9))
 (segment (start 56.385 76.655) (end 56.385 73.535) (width 1.5) (layer "B.Cu") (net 9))
 (segment (start 61 68.92) (end 67 68.92) (width 1.5) (layer "B.Cu") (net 9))
 (segment (start 80 68.92) (end 82 66.92) (width 1.5) (layer "B.Cu") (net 9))
 (segment (start 67 68.92) (end 80 68.92) (width 1.5) (layer "B.Cu") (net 9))
 (segment (start 82 66.92) (end 82 63.7) (width 1.5) (layer "B.Cu") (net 9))
 (segment (start 67 33.46) (end 61.46 33.46) (width 1) (layer "B.Cu") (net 4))
 (segment (start 74.62 28.38) (end 74.62 25.84) (width 1) (layer "B.Cu") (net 4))
 (segment (start 61.46 33.46) (end 46.46 18.46) (width 1) (layer "B.Cu") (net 4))
 (segment (start 46.46 18.46) (end 43 18.46) (width 1) (layer "B.Cu") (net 4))
 (segment (start 60 54.46) (end 62.54 57) (width 1) (layer "B.Cu") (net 14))
 (segment (start 64.24 58.7) (end 62.54 57) (width 1) (layer "B.Cu") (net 14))
 (segment (start 82 58.7) (end 64.24 58.7) (width 1) (layer "B.Cu") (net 14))
 (segment (start 60.92 51) (end 60 51.92) (width 1) (layer "B.Cu") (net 13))
 (segment (start 82 51) (end 60.92 51) (width 1) (layer "B.Cu") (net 13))
 (segment (start 67 25.84) (end 67 23.3) (width 1) (layer "B.Cu") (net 1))
 (segment (start 71 34) (end 73 36) (width 1) (layer "B.Cu") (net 1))
 (segment (start 119 31.08) (end 119 40) (width 1) (layer "B.Cu") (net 1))
 (segment (start 67 25.84) (end 68.84 25.84) (width 1) (layer "B.Cu") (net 1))
 (segment (start 68.84 25.84) (end 71 28) (width 1) (layer "B.Cu") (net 1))
 (segment (start 81 36) (end 74.62 36) (width 1) (layer "B.Cu") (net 1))
 (segment (start 126 24.08) (end 119 31.08) (width 1) (layer "B.Cu") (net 1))
 (segment (start 73 36) (end 74.62 36) (width 1) (layer "B.Cu") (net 1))
 (segment (start 119 40) (end 116 43) (width 1) (layer "B.Cu") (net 1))
 (segment (start 88 43) (end 81 36) (width 1) (layer "B.Cu") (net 1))
 (segment (start 116 43) (end 88 43) (width 1) (layer "B.Cu") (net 1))
 (segment (start 71 28) (end 71 34) (width 1) (layer "B.Cu") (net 1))
 (segment (start 89.62 58.62) (end 109.3 58.62) (width 1.5) (layer "B.Cu") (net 10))
 (segment (start 109.3 58.62) (end 111 56.92) (width 1.5) (layer "B.Cu") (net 10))
 (segment (start 111 56.92) (end 111 54.46) (width 1.5) (layer "B.Cu") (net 10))
 (segment (start 89.62 51) (end 110.08 51) (width 1) (layer "B.Cu") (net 11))
 (segment (start 110.08 51) (end 111 51.92) (width 1) (layer "B.Cu") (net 11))
 (segment (start 95 18) (end 96.38 19.38) (width 1) (layer "B.Cu") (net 6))
 (segment (start 61.92 30.92) (end 60 29) (width 1) (layer "B.Cu") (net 6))
 (segment (start 96.38 19.38) (end 96.38 21) (width 1) (layer "B.Cu") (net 6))
 (segment (start 60 29) (end 60 23) (width 1) (layer "B.Cu") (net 6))
 (segment (start 67 20.76) (end 67 19) (width 1) (layer "B.Cu") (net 6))
 (segment (start 62.24 20.76) (end 67 20.76) (width 1) (layer "B.Cu") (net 6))
 (segment (start 67 30.92) (end 61.92 30.92) (width 1) (layer "B.Cu") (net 6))
 (segment (start 68 18) (end 95 18) (width 1) (layer "B.Cu") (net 6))
 (segment (start 60 23) (end 62.24 20.76) (width 1) (layer "B.Cu") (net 6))
 (segment (start 67 19) (end 68 18) (width 1) (layer "B.Cu") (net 6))
 (segment (start 74.62 30.92) (end 78 30.92) (width 1.5) (layer "B.Cu") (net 3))
 (segment (start 104 23.54) (end 108.54 23.54) (width 1.5) (layer "B.Cu") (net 3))
 (segment (start 67 28.38) (end 63 28.38) (width 1.5) (layer "B.Cu") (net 7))
 (segment (start 63 28.38) (end 63.62 28.38) (width 1) (layer "B.Cu") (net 7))
 (segment (start 96.38 31.16) (end 94.16 31.16) (width 1.5) (layer "B.Cu") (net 7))
 (segment (start 82 48.54) (end 76.54 48.54) (width 1.5) (layer "B.Cu") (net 12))
 (segment (start 96.38 26.08) (end 96.38 28.62) (width 1) (layer "B.Cu") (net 12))
 (segment (start 104 31.16) (end 104 28.62) (width 1) (layer "B.Cu") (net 17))
 (segment (start 92.46 23.54) (end 96.38 23.54) (width 1) (layer "B.Cu") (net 16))
 (segment (start 93.7 33.7) (end 91 31) (width 1) (layer "B.Cu") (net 16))
 (segment (start 96.38 33.7) (end 93.7 33.7) (width 1) (layer "B.Cu") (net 16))
 (segment (start 91 31) (end 91 25) (width 1) (layer "B.Cu") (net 16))
 (segment (start 91 25) (end 92.46 23.54) (width 1) (layer "B.Cu") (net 16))
 (segment (start 101 35) (end 101 27) (width 1) (layer "B.Cu") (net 15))
 (segment (start 102.24 36.24) (end 101 35) (width 1) (layer "B.Cu") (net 15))
 (segment (start 104 36.24) (end 102.24 36.24) (width 1) (layer "B.Cu") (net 15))
 (segment (start 101 27) (end 101.92 26.08) (width 1) (layer "B.Cu") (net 15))
 (segment (start 101.92 26.08) (end 104 26.08) (width 1) (layer "B.Cu") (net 15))
 (segment (start 76.3 23.3) (end 74.62 23.3) (width 1) (layer "B.Cu") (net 2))
 (segment (start 91 40) (end 84.46 33.46) (width 1) (layer "B.Cu") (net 2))
 (segment (start 91 40) (end 107 40) (width 1) (layer "B.Cu") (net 2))
 (segment (start 81 30) (end 81 28) (width 1) (layer "B.Cu") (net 2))
 (segment (start 109 35) (end 107.7 33.7) (width 1) (layer "B.Cu") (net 2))
 (segment (start 84.46 33.46) (end 81 30) (width 1) (layer "B.Cu") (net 2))
 (segment (start 104 33.7) (end 107.7 33.7) (width 1) (layer "B.Cu") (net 2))
 (segment (start 109 38) (end 109 35) (width 1) (layer "B.Cu") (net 2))
 (segment (start 107 40) (end 109 38) (width 1) (layer "B.Cu") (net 2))
 (segment (start 84.46 33.46) (end 74.62 33.46) (width 1) (layer "B.Cu") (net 2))
 (segment (start 74.62 33.46) (end 76.54 33.46) (width 1) (layer "B.Cu") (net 2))
 (segment (start 81 28) (end 76.3 23.3) (width 1) (layer "B.Cu") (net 2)))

